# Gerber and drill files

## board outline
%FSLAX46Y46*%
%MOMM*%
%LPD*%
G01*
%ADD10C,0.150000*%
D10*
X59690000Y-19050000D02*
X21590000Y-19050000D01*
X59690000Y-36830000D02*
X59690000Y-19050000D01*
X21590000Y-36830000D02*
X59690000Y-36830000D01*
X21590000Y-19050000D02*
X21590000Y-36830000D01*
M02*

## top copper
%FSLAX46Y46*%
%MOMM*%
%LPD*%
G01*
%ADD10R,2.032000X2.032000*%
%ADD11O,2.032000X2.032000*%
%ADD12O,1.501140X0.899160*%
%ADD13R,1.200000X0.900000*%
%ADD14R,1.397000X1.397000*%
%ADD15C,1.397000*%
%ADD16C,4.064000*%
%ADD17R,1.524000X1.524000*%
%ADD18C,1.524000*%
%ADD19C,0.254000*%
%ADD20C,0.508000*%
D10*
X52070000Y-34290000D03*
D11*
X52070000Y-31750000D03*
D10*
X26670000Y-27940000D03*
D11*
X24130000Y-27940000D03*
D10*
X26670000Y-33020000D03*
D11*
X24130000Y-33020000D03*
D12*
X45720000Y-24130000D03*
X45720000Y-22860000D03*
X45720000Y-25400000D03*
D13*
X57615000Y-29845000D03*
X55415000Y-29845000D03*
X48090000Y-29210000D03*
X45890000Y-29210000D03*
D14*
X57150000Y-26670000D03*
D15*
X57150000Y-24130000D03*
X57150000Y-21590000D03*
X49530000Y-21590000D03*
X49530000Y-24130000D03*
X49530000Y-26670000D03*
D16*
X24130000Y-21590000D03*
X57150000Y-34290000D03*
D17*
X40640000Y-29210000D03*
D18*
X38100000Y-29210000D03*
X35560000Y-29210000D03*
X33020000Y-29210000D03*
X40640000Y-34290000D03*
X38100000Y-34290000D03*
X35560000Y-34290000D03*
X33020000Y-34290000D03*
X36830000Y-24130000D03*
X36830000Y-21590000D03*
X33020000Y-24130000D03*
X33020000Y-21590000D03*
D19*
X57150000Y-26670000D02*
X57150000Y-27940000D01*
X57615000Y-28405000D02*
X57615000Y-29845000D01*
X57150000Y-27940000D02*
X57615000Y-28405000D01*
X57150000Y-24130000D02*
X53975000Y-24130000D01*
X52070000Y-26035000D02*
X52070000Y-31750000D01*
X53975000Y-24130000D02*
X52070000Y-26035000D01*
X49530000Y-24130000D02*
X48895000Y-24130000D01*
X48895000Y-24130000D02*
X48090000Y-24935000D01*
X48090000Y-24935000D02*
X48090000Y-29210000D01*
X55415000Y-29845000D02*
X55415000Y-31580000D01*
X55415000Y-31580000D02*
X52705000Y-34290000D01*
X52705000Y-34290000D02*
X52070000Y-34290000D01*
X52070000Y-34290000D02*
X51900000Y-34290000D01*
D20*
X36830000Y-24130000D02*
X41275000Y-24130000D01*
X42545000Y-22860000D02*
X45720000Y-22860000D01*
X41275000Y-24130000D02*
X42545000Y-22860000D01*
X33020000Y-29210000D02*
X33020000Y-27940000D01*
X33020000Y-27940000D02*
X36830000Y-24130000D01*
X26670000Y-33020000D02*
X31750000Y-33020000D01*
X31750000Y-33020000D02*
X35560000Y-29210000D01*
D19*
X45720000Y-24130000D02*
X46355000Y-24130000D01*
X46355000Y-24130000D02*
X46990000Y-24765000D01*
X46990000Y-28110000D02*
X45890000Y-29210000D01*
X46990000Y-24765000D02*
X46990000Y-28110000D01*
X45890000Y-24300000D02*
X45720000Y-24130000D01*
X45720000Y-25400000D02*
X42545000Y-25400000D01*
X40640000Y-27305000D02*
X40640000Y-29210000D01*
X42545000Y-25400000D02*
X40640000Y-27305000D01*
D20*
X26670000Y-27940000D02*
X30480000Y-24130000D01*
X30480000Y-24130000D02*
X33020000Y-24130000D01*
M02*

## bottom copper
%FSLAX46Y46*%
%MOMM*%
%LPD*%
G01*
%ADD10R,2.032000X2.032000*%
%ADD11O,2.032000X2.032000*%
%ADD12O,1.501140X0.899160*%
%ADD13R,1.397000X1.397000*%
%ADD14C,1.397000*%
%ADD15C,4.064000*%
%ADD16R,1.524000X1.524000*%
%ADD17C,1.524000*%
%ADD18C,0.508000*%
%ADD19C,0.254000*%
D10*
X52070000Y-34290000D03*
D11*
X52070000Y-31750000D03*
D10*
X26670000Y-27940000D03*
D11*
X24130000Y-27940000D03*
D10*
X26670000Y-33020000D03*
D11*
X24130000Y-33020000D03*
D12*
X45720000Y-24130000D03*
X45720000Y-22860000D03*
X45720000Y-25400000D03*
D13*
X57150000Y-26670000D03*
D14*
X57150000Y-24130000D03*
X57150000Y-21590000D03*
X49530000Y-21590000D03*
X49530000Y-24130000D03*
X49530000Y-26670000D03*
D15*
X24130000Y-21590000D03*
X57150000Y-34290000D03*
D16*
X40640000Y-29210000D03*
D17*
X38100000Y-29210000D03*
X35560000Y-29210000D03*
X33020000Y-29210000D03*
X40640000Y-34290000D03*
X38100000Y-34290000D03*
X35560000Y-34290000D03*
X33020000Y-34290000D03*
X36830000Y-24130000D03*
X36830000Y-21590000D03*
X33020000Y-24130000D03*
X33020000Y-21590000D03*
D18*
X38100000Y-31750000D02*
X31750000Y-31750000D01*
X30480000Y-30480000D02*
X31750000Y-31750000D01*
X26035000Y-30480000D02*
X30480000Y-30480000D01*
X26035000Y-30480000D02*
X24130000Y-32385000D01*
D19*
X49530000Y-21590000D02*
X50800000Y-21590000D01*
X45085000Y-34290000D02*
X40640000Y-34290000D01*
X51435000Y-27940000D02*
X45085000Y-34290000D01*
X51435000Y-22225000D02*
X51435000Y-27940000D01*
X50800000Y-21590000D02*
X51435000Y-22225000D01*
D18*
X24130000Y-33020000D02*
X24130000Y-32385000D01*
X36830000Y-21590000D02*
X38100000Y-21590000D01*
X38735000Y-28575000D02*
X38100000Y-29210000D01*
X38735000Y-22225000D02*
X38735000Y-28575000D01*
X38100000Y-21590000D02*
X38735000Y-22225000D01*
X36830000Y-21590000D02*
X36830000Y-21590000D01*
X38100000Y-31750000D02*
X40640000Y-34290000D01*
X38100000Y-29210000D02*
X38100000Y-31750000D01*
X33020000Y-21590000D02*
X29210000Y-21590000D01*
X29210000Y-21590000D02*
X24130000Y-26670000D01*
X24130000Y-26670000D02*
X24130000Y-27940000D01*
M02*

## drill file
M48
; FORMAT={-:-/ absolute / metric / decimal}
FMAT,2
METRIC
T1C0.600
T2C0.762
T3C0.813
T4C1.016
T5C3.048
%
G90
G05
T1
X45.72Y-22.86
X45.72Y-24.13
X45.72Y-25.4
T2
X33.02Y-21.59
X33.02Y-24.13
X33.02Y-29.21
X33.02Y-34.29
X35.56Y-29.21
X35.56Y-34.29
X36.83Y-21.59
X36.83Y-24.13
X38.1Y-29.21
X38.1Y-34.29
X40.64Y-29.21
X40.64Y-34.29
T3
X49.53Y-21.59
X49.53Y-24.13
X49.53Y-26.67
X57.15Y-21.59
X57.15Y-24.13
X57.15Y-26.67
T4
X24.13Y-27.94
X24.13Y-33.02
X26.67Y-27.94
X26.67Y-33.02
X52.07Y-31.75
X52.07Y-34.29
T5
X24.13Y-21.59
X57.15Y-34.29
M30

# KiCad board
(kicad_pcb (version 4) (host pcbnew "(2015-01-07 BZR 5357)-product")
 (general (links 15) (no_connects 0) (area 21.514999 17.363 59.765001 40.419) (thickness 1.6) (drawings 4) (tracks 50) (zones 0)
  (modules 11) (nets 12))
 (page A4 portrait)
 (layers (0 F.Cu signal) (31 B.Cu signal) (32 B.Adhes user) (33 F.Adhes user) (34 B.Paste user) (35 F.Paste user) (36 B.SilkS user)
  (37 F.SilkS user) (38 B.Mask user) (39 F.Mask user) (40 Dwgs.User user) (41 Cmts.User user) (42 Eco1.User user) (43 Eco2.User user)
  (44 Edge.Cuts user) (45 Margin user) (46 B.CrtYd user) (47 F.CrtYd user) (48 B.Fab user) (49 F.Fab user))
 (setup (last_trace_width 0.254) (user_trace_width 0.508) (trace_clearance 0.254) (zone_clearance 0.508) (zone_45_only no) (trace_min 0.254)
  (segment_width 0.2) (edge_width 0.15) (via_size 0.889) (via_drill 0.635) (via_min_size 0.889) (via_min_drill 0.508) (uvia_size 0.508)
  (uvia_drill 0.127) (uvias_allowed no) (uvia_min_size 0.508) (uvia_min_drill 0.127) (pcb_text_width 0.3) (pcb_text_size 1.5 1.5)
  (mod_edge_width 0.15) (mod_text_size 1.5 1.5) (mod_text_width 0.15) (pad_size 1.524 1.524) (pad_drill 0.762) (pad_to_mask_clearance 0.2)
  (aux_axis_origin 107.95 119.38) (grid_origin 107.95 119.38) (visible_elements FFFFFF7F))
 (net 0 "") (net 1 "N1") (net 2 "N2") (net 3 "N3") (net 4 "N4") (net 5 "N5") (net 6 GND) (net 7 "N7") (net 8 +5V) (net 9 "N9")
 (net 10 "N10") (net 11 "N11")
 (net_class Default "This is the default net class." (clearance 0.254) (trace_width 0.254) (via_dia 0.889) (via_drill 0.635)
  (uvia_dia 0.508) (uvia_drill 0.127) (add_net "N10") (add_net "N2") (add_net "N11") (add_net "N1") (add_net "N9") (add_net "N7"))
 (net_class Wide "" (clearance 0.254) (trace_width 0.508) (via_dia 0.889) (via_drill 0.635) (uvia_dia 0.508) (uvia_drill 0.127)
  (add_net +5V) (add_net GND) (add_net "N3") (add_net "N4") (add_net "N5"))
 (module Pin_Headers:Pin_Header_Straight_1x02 (layer F.Cu) (at 52.07 34.29 180)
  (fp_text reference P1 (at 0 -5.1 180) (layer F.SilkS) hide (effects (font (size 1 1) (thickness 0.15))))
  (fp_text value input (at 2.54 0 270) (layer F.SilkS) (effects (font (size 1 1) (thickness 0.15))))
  (pad 1 thru_hole rect (at 0 0 180) (size 2.032 2.032) (drill 1.016) (layers *.Cu *.Mask F.SilkS) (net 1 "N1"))
  (pad 2 thru_hole oval (at 0 2.54 180) (size 2.032 2.032) (drill 1.016) (layers *.Cu *.Mask F.SilkS) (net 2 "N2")))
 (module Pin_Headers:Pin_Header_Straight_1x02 (layer F.Cu) (at 26.67 27.94 270)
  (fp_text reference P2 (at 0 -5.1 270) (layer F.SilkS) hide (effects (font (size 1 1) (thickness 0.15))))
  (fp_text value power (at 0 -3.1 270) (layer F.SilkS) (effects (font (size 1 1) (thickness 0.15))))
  (pad 1 thru_hole rect (at 0 0 270) (size 2.032 2.032) (drill 1.016) (layers *.Cu *.Mask F.SilkS) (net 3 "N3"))
  (pad 2 thru_hole oval (at 0 2.54 270) (size 2.032 2.032) (drill 1.016) (layers *.Cu *.Mask F.SilkS) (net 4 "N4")))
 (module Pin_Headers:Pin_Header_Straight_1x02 (layer F.Cu) (at 26.67 33.02 270)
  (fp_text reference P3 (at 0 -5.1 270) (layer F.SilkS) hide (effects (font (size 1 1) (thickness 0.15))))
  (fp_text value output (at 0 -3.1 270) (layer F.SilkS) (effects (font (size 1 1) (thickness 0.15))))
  (pad 1 thru_hole rect (at 0 0 270) (size 2.032 2.032) (drill 1.016) (layers *.Cu *.Mask F.SilkS) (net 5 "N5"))
  (pad 2 thru_hole oval (at 0 2.54 270) (size 2.032 2.032) (drill 1.016) (layers *.Cu *.Mask F.SilkS) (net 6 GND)))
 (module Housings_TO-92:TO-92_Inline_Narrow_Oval (layer F.Cu) (at 45.72 25.4 90)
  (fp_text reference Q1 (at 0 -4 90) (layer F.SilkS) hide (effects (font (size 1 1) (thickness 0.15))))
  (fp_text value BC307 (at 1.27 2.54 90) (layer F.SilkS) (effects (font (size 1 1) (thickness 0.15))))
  (pad 2 thru_hole oval (at 1.27 0 270) (size 0.89916 1.50114) (drill 0.6) (layers *.Cu *.Mask F.SilkS) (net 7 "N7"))
  (pad 3 thru_hole oval (at 2.54 0 270) (size 0.89916 1.50114) (drill 0.6) (layers *.Cu *.Mask F.SilkS) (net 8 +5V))
  (pad 1 thru_hole oval (at 0 0 270) (size 0.89916 1.50114) (drill 0.6) (layers *.Cu *.Mask F.SilkS) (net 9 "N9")))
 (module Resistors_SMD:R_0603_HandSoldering (layer F.Cu) (at 56.515 29.845 180)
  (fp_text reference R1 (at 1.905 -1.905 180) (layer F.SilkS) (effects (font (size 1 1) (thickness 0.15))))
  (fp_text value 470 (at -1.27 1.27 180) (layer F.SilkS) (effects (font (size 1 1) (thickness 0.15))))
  (pad 1 smd rect (at -1.1 0 180) (size 1.2 0.9) (layers F.Cu F.Paste F.Mask) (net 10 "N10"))
  (pad 2 smd rect (at 1.1 0 180) (size 1.2 0.9) (layers F.Cu F.Paste F.Mask) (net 1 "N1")))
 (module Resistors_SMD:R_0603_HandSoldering (layer F.Cu) (at 46.99 29.21 180)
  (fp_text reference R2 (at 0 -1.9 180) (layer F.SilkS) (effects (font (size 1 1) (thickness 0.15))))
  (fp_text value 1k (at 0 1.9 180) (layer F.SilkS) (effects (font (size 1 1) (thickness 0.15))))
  (pad 1 smd rect (at -1.1 0 180) (size 1.2 0.9) (layers F.Cu F.Paste F.Mask) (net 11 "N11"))
  (pad 2 smd rect (at 1.1 0 180) (size 1.2 0.9) (layers F.Cu F.Paste F.Mask) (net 7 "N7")))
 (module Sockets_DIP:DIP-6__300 (layer F.Cu) (at 53.34 24.13 90)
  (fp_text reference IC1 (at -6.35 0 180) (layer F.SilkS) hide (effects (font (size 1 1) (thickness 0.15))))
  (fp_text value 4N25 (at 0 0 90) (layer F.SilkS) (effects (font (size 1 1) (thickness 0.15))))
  (pad 1 thru_hole rect (at -2.54 3.81 90) (size 1.397 1.397) (drill 0.8128) (layers *.Cu *.Mask F.SilkS) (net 10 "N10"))
  (pad 2 thru_hole circle (at 0 3.81 90) (size 1.397 1.397) (drill 0.8128) (layers *.Cu *.Mask F.SilkS) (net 2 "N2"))
  (pad 3 thru_hole circle (at 2.54 3.81 90) (size 1.397 1.397) (drill 0.8128) (layers *.Cu *.Mask F.SilkS))
  (pad 4 thru_hole circle (at 2.54 -3.81 90) (size 1.397 1.397) (drill 0.8128) (layers *.Cu *.Mask F.SilkS) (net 6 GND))
  (pad 5 thru_hole circle (at 0 -3.81 90) (size 1.397 1.397) (drill 0.8128) (layers *.Cu *.Mask F.SilkS) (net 11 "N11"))
  (pad 6 thru_hole circle (at -2.54 -3.81 90) (size 1.397 1.397) (drill 0.8128) (layers *.Cu *.Mask F.SilkS)))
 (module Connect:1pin (layer F.Cu) (at 24.13 21.59)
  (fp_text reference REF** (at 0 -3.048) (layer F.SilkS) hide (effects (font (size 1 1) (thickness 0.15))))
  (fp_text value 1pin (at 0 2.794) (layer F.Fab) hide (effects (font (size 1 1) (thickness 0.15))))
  (pad 1 thru_hole circle (at 0 0) (size 4.064 4.064) (drill 3.048) (layers *.Cu *.Mask F.SilkS)))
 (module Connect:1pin (layer F.Cu) (at 57.15 34.29)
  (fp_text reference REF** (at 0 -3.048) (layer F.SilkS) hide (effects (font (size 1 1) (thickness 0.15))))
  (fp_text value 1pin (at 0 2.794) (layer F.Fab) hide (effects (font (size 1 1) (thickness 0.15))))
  (pad 1 thru_hole circle (at 0 0) (size 4.064 4.064) (drill 3.048) (layers *.Cu *.Mask F.SilkS)))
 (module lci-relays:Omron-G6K (layer F.Cu) (at 36.83 31.75 180)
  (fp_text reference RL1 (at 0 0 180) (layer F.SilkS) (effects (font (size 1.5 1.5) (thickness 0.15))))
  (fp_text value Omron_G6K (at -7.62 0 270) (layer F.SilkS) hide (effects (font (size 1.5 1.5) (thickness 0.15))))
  (pad 1 thru_hole rect (at -3.81 2.54 180) (size 1.524 1.524) (drill 0.762) (layers *.Cu *.Mask F.SilkS) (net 9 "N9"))
  (pad 2 thru_hole circle (at -1.27 2.54 180) (size 1.524 1.524) (drill 0.762) (layers *.Cu *.Mask F.SilkS) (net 6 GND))
  (pad 3 thru_hole circle (at 1.27 2.54 180) (size 1.524 1.524) (drill 0.762) (layers *.Cu *.Mask F.SilkS) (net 5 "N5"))
  (pad 4 thru_hole circle (at 3.81 2.54 180) (size 1.524 1.524) (drill 0.762) (layers *.Cu *.Mask F.SilkS) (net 8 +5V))
  (pad 8 thru_hole circle (at -3.81 -2.54 180) (size 1.524 1.524) (drill 0.762) (layers *.Cu *.Mask F.SilkS) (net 6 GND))
  (pad 7 thru_hole circle (at -1.27 -2.54 180) (size 1.524 1.524) (drill 0.762) (layers *.Cu *.Mask F.SilkS))
  (pad 6 thru_hole circle (at 1.27 -2.54 180) (size 1.524 1.524) (drill 0.762) (layers *.Cu *.Mask F.SilkS))
  (pad 5 thru_hole circle (at 3.81 -2.54 180) (size 1.524 1.524) (drill 0.762) (layers *.Cu *.Mask F.SilkS)))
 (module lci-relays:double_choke (layer F.Cu) (at 34.29 22.86 180)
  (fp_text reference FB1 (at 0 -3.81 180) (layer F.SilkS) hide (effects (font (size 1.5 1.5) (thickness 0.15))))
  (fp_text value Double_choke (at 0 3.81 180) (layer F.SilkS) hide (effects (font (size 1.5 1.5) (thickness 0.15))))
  (pad 1 thru_hole circle (at -2.54 -1.27 180) (size 1.524 1.524) (drill 0.762) (layers *.Cu *.Mask F.SilkS) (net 8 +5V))
  (pad 2 thru_hole circle (at -2.54 1.27 180) (size 1.524 1.524) (drill 0.762) (layers *.Cu *.Mask F.SilkS) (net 6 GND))
  (pad 3 thru_hole circle (at 1.27 -1.27 180) (size 1.524 1.524) (drill 0.762) (layers *.Cu *.Mask F.SilkS) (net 3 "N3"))
  (pad 4 thru_hole circle (at 1.27 1.27 180) (size 1.524 1.524) (drill 0.762) (layers *.Cu *.Mask F.SilkS) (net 4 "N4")))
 (gr_line (start 59.69 19.05) (end 21.59 19.05) (angle 90) (layer Edge.Cuts) (width 0.15))
 (gr_line (start 59.69 36.83) (end 59.69 19.05) (angle 90) (layer Edge.Cuts) (width 0.15))
 (gr_line (start 21.59 36.83) (end 59.69 36.83) (angle 90) (layer Edge.Cuts) (width 0.15))
 (gr_line (start 21.59 19.05) (end 21.59 36.83) (angle 90) (layer Edge.Cuts) (width 0.15))
 (segment (start 57.15 26.67) (end 57.15 27.94) (width 0.254) (layer F.Cu) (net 10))
 (segment (start 57.615 28.405) (end 57.615 29.845) (width 0.254) (layer F.Cu) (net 10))
 (segment (start 57.15 27.94) (end 57.615 28.405) (width 0.254) (layer F.Cu) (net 10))
 (segment (start 57.15 24.13) (end 53.975 24.13) (width 0.254) (layer F.Cu) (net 2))
 (segment (start 52.07 26.035) (end 52.07 31.75) (width 0.254) (layer F.Cu) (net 2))
 (segment (start 53.975 24.13) (end 52.07 26.035) (width 0.254) (layer F.Cu) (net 2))
 (segment (start 38.1 31.75) (end 31.75 31.75) (width 0.508) (layer B.Cu) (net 6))
 (segment (start 30.48 30.48) (end 31.75 31.75) (width 0.508) (layer B.Cu) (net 6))
 (segment (start 26.035 30.48) (end 30.48 30.48) (width 0.508) (layer B.Cu) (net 6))
 (segment (start 26.035 30.48) (end 24.13 32.385) (width 0.508) (layer B.Cu) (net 6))
 (segment (start 49.53 21.59) (end 50.8 21.59) (width 0.254) (layer B.Cu) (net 6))
 (segment (start 45.085 34.29) (end 40.64 34.29) (width 0.254) (layer B.Cu) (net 6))
 (segment (start 51.435 27.94) (end 45.085 34.29) (width 0.254) (layer B.Cu) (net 6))
 (segment (start 51.435 22.225) (end 51.435 27.94) (width 0.254) (layer B.Cu) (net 6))
 (segment (start 50.8 21.59) (end 51.435 22.225) (width 0.254) (layer B.Cu) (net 6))
 (segment (start 24.13 33.02) (end 24.13 32.385) (width 0.508) (layer B.Cu) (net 6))
 (segment (start 36.83 21.59) (end 38.1 21.59) (width 0.508) (layer B.Cu) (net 6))
 (segment (start 38.735 28.575) (end 38.1 29.21) (width 0.508) (layer B.Cu) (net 6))
 (segment (start 38.735 22.225) (end 38.735 28.575) (width 0.508) (layer B.Cu) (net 6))
 (segment (start 38.1 21.59) (end 38.735 22.225) (width 0.508) (layer B.Cu) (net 6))
 (segment (start 36.83 21.59) (end 36.83 21.59) (width 0.508) (layer B.Cu) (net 6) (status 30))
 (segment (start 38.1 31.75) (end 40.64 34.29) (width 0.508) (layer B.Cu) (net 6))
 (segment (start 38.1 29.21) (end 38.1 31.75) (width 0.508) (layer B.Cu) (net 6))
 (segment (start 49.53 24.13) (end 48.895 24.13) (width 0.254) (layer F.Cu) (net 11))
 (segment (start 48.895 24.13) (end 48.09 24.935) (width 0.254) (layer F.Cu) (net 11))
 (segment (start 48.09 24.935) (end 48.09 29.21) (width 0.254) (layer F.Cu) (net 11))
 (segment (start 55.415 29.845) (end 55.415 31.58) (width 0.254) (layer F.Cu) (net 1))
 (segment (start 55.415 31.58) (end 52.705 34.29) (width 0.254) (layer F.Cu) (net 1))
 (segment (start 52.705 34.29) (end 52.07 34.29) (width 0.254) (layer F.Cu) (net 1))
 (segment (start 52.07 34.29) (end 51.9 34.29) (width 0.254) (layer F.Cu) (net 1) (status 30))
 (segment (start 36.83 24.13) (end 41.275 24.13) (width 0.508) (layer F.Cu) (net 8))
 (segment (start 42.545 22.86) (end 45.72 22.86) (width 0.508) (layer F.Cu) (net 8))
 (segment (start 41.275 24.13) (end 42.545 22.86) (width 0.508) (layer F.Cu) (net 8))
 (segment (start 33.02 29.21) (end 33.02 27.94) (width 0.508) (layer F.Cu) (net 8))
 (segment (start 33.02 27.94) (end 36.83 24.13) (width 0.508) (layer F.Cu) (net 8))
 (segment (start 26.67 33.02) (end 31.75 33.02) (width 0.508) (layer F.Cu) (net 5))
 (segment (start 31.75 33.02) (end 35.56 29.21) (width 0.508) (layer F.Cu) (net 5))
 (segment (start 45.72 24.13) (end 46.355 24.13) (width 0.254) (layer F.Cu) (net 7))
 (segment (start 46.355 24.13) (end 46.99 24.765) (width 0.254) (layer F.Cu) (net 7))
 (segment (start 46.99 28.11) (end 45.89 29.21) (width 0.254) (layer F.Cu) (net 7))
 (segment (start 46.99 24.765) (end 46.99 28.11) (width 0.254) (layer F.Cu) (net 7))
 (segment (start 45.89 24.3) (end 45.72 24.13) (width 0.254) (layer F.Cu) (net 7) (status 30))
 (segment (start 45.72 25.4) (end 42.545 25.4) (width 0.254) (layer F.Cu) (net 9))
 (segment (start 40.64 27.305) (end 40.64 29.21) (width 0.254) (layer F.Cu) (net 9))
 (segment (start 42.545 25.4) (end 40.64 27.305) (width 0.254) (layer F.Cu) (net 9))
 (segment (start 26.67 27.94) (end 30.48 24.13) (width 0.508) (layer F.Cu) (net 3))
 (segment (start 30.48 24.13) (end 33.02 24.13) (width 0.508) (layer F.Cu) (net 3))
 (segment (start 33.02 21.59) (end 29.21 21.59) (width 0.508) (layer B.Cu) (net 4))
 (segment (start 29.21 21.59) (end 24.13 26.67) (width 0.508) (layer B.Cu) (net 4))
 (segment (start 24.13 26.67) (end 24.13 27.94) (width 0.508) (layer B.Cu) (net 4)))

